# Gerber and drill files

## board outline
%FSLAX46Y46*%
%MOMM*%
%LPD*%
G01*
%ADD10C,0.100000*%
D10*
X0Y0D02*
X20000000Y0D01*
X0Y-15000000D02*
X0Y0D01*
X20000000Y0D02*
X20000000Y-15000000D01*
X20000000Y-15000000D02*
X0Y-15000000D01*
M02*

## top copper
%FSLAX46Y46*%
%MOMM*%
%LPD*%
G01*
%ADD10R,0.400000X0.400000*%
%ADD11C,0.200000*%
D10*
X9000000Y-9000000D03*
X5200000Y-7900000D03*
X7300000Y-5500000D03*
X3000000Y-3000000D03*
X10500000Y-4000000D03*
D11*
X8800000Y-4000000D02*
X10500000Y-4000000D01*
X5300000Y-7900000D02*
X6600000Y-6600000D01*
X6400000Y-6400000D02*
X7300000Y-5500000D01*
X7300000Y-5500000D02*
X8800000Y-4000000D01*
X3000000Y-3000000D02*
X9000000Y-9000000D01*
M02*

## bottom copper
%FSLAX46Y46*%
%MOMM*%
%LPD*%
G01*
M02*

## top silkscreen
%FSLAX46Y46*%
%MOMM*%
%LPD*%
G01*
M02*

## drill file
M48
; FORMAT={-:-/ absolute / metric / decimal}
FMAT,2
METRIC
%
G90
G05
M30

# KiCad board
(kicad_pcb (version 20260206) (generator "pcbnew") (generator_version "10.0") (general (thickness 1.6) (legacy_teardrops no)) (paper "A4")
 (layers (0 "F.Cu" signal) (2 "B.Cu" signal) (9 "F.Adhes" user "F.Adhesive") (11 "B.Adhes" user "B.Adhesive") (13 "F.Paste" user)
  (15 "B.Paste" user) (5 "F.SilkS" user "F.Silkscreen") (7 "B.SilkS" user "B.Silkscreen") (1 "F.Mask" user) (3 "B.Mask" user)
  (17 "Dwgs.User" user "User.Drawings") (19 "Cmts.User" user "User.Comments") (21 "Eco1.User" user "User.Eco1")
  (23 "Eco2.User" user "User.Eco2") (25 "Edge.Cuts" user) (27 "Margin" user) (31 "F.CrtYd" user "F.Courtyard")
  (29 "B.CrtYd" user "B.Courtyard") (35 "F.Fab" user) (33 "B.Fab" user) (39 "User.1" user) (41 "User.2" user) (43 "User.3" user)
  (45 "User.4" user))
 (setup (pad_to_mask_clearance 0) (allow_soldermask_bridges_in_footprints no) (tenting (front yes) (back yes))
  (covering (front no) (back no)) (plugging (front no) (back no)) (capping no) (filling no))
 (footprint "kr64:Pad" (layer "F.Cu") (at 9 9)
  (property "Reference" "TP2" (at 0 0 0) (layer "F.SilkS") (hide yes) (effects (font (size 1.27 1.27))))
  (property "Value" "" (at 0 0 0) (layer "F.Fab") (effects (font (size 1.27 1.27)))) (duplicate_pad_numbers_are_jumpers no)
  (pad "1" smd rect (at 0 0) (size 0.4 0.4) (layers "F.Cu" "F.Mask" "F.Paste") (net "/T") (thermal_bridge_angle 45)))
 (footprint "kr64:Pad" (layer "F.Cu") (at 5.2 7.9)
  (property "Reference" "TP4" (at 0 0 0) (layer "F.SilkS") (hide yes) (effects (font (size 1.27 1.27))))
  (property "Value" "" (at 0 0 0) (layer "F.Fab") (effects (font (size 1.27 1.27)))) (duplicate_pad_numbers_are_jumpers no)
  (pad "1" smd rect (at 0 0) (size 0.4 0.4) (layers "F.Cu" "F.Mask" "F.Paste") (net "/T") (thermal_bridge_angle 45)))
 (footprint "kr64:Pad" (layer "F.Cu") (at 7.3 5.5)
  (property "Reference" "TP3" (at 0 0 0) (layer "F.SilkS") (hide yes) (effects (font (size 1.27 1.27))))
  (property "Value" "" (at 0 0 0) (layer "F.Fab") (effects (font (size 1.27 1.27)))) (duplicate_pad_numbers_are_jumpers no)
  (pad "1" smd rect (at 0 0) (size 0.4 0.4) (layers "F.Cu" "F.Mask" "F.Paste") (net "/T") (thermal_bridge_angle 45)))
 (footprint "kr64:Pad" (layer "F.Cu") (at 3 3)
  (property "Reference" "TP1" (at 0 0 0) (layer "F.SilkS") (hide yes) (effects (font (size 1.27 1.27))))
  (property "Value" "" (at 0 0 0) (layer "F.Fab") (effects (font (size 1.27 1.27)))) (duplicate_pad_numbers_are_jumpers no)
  (pad "1" smd rect (at 0 0) (size 0.4 0.4) (layers "F.Cu" "F.Mask" "F.Paste") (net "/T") (thermal_bridge_angle 45)))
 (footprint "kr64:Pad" (layer "F.Cu") (at 10.5 4)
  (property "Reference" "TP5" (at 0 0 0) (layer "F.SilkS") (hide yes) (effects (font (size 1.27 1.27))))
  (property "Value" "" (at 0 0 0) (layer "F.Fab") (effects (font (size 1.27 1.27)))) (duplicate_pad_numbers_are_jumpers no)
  (pad "1" smd rect (at 0 0) (size 0.4 0.4) (layers "F.Cu" "F.Mask" "F.Paste") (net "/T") (thermal_bridge_angle 45)))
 (gr_line (start 0 0) (end 20 0) (stroke (width 0.1) (type default)) (layer "Edge.Cuts"))
 (gr_line (start 0 15) (end 0 0) (stroke (width 0.1) (type default)) (layer "Edge.Cuts"))
 (gr_line (start 20 0) (end 20 15) (stroke (width 0.1) (type default)) (layer "Edge.Cuts"))
 (gr_line (start 20 15) (end 0 15) (stroke (width 0.1) (type default)) (layer "Edge.Cuts"))
 (segment (start 8.8 4) (end 10.5 4) (width 0.2) (layer "F.Cu") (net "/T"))
 (segment (start 5.3 7.9) (end 6.6 6.6) (width 0.2) (layer "F.Cu") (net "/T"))
 (segment (start 6.4 6.4) (end 7.3 5.5) (width 0.2) (layer "F.Cu") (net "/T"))
 (segment (start 7.3 5.5) (end 8.8 4) (width 0.2) (layer "F.Cu") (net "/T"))
 (segment (start 3 3) (end 9 9) (width 0.2) (layer "F.Cu") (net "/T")))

